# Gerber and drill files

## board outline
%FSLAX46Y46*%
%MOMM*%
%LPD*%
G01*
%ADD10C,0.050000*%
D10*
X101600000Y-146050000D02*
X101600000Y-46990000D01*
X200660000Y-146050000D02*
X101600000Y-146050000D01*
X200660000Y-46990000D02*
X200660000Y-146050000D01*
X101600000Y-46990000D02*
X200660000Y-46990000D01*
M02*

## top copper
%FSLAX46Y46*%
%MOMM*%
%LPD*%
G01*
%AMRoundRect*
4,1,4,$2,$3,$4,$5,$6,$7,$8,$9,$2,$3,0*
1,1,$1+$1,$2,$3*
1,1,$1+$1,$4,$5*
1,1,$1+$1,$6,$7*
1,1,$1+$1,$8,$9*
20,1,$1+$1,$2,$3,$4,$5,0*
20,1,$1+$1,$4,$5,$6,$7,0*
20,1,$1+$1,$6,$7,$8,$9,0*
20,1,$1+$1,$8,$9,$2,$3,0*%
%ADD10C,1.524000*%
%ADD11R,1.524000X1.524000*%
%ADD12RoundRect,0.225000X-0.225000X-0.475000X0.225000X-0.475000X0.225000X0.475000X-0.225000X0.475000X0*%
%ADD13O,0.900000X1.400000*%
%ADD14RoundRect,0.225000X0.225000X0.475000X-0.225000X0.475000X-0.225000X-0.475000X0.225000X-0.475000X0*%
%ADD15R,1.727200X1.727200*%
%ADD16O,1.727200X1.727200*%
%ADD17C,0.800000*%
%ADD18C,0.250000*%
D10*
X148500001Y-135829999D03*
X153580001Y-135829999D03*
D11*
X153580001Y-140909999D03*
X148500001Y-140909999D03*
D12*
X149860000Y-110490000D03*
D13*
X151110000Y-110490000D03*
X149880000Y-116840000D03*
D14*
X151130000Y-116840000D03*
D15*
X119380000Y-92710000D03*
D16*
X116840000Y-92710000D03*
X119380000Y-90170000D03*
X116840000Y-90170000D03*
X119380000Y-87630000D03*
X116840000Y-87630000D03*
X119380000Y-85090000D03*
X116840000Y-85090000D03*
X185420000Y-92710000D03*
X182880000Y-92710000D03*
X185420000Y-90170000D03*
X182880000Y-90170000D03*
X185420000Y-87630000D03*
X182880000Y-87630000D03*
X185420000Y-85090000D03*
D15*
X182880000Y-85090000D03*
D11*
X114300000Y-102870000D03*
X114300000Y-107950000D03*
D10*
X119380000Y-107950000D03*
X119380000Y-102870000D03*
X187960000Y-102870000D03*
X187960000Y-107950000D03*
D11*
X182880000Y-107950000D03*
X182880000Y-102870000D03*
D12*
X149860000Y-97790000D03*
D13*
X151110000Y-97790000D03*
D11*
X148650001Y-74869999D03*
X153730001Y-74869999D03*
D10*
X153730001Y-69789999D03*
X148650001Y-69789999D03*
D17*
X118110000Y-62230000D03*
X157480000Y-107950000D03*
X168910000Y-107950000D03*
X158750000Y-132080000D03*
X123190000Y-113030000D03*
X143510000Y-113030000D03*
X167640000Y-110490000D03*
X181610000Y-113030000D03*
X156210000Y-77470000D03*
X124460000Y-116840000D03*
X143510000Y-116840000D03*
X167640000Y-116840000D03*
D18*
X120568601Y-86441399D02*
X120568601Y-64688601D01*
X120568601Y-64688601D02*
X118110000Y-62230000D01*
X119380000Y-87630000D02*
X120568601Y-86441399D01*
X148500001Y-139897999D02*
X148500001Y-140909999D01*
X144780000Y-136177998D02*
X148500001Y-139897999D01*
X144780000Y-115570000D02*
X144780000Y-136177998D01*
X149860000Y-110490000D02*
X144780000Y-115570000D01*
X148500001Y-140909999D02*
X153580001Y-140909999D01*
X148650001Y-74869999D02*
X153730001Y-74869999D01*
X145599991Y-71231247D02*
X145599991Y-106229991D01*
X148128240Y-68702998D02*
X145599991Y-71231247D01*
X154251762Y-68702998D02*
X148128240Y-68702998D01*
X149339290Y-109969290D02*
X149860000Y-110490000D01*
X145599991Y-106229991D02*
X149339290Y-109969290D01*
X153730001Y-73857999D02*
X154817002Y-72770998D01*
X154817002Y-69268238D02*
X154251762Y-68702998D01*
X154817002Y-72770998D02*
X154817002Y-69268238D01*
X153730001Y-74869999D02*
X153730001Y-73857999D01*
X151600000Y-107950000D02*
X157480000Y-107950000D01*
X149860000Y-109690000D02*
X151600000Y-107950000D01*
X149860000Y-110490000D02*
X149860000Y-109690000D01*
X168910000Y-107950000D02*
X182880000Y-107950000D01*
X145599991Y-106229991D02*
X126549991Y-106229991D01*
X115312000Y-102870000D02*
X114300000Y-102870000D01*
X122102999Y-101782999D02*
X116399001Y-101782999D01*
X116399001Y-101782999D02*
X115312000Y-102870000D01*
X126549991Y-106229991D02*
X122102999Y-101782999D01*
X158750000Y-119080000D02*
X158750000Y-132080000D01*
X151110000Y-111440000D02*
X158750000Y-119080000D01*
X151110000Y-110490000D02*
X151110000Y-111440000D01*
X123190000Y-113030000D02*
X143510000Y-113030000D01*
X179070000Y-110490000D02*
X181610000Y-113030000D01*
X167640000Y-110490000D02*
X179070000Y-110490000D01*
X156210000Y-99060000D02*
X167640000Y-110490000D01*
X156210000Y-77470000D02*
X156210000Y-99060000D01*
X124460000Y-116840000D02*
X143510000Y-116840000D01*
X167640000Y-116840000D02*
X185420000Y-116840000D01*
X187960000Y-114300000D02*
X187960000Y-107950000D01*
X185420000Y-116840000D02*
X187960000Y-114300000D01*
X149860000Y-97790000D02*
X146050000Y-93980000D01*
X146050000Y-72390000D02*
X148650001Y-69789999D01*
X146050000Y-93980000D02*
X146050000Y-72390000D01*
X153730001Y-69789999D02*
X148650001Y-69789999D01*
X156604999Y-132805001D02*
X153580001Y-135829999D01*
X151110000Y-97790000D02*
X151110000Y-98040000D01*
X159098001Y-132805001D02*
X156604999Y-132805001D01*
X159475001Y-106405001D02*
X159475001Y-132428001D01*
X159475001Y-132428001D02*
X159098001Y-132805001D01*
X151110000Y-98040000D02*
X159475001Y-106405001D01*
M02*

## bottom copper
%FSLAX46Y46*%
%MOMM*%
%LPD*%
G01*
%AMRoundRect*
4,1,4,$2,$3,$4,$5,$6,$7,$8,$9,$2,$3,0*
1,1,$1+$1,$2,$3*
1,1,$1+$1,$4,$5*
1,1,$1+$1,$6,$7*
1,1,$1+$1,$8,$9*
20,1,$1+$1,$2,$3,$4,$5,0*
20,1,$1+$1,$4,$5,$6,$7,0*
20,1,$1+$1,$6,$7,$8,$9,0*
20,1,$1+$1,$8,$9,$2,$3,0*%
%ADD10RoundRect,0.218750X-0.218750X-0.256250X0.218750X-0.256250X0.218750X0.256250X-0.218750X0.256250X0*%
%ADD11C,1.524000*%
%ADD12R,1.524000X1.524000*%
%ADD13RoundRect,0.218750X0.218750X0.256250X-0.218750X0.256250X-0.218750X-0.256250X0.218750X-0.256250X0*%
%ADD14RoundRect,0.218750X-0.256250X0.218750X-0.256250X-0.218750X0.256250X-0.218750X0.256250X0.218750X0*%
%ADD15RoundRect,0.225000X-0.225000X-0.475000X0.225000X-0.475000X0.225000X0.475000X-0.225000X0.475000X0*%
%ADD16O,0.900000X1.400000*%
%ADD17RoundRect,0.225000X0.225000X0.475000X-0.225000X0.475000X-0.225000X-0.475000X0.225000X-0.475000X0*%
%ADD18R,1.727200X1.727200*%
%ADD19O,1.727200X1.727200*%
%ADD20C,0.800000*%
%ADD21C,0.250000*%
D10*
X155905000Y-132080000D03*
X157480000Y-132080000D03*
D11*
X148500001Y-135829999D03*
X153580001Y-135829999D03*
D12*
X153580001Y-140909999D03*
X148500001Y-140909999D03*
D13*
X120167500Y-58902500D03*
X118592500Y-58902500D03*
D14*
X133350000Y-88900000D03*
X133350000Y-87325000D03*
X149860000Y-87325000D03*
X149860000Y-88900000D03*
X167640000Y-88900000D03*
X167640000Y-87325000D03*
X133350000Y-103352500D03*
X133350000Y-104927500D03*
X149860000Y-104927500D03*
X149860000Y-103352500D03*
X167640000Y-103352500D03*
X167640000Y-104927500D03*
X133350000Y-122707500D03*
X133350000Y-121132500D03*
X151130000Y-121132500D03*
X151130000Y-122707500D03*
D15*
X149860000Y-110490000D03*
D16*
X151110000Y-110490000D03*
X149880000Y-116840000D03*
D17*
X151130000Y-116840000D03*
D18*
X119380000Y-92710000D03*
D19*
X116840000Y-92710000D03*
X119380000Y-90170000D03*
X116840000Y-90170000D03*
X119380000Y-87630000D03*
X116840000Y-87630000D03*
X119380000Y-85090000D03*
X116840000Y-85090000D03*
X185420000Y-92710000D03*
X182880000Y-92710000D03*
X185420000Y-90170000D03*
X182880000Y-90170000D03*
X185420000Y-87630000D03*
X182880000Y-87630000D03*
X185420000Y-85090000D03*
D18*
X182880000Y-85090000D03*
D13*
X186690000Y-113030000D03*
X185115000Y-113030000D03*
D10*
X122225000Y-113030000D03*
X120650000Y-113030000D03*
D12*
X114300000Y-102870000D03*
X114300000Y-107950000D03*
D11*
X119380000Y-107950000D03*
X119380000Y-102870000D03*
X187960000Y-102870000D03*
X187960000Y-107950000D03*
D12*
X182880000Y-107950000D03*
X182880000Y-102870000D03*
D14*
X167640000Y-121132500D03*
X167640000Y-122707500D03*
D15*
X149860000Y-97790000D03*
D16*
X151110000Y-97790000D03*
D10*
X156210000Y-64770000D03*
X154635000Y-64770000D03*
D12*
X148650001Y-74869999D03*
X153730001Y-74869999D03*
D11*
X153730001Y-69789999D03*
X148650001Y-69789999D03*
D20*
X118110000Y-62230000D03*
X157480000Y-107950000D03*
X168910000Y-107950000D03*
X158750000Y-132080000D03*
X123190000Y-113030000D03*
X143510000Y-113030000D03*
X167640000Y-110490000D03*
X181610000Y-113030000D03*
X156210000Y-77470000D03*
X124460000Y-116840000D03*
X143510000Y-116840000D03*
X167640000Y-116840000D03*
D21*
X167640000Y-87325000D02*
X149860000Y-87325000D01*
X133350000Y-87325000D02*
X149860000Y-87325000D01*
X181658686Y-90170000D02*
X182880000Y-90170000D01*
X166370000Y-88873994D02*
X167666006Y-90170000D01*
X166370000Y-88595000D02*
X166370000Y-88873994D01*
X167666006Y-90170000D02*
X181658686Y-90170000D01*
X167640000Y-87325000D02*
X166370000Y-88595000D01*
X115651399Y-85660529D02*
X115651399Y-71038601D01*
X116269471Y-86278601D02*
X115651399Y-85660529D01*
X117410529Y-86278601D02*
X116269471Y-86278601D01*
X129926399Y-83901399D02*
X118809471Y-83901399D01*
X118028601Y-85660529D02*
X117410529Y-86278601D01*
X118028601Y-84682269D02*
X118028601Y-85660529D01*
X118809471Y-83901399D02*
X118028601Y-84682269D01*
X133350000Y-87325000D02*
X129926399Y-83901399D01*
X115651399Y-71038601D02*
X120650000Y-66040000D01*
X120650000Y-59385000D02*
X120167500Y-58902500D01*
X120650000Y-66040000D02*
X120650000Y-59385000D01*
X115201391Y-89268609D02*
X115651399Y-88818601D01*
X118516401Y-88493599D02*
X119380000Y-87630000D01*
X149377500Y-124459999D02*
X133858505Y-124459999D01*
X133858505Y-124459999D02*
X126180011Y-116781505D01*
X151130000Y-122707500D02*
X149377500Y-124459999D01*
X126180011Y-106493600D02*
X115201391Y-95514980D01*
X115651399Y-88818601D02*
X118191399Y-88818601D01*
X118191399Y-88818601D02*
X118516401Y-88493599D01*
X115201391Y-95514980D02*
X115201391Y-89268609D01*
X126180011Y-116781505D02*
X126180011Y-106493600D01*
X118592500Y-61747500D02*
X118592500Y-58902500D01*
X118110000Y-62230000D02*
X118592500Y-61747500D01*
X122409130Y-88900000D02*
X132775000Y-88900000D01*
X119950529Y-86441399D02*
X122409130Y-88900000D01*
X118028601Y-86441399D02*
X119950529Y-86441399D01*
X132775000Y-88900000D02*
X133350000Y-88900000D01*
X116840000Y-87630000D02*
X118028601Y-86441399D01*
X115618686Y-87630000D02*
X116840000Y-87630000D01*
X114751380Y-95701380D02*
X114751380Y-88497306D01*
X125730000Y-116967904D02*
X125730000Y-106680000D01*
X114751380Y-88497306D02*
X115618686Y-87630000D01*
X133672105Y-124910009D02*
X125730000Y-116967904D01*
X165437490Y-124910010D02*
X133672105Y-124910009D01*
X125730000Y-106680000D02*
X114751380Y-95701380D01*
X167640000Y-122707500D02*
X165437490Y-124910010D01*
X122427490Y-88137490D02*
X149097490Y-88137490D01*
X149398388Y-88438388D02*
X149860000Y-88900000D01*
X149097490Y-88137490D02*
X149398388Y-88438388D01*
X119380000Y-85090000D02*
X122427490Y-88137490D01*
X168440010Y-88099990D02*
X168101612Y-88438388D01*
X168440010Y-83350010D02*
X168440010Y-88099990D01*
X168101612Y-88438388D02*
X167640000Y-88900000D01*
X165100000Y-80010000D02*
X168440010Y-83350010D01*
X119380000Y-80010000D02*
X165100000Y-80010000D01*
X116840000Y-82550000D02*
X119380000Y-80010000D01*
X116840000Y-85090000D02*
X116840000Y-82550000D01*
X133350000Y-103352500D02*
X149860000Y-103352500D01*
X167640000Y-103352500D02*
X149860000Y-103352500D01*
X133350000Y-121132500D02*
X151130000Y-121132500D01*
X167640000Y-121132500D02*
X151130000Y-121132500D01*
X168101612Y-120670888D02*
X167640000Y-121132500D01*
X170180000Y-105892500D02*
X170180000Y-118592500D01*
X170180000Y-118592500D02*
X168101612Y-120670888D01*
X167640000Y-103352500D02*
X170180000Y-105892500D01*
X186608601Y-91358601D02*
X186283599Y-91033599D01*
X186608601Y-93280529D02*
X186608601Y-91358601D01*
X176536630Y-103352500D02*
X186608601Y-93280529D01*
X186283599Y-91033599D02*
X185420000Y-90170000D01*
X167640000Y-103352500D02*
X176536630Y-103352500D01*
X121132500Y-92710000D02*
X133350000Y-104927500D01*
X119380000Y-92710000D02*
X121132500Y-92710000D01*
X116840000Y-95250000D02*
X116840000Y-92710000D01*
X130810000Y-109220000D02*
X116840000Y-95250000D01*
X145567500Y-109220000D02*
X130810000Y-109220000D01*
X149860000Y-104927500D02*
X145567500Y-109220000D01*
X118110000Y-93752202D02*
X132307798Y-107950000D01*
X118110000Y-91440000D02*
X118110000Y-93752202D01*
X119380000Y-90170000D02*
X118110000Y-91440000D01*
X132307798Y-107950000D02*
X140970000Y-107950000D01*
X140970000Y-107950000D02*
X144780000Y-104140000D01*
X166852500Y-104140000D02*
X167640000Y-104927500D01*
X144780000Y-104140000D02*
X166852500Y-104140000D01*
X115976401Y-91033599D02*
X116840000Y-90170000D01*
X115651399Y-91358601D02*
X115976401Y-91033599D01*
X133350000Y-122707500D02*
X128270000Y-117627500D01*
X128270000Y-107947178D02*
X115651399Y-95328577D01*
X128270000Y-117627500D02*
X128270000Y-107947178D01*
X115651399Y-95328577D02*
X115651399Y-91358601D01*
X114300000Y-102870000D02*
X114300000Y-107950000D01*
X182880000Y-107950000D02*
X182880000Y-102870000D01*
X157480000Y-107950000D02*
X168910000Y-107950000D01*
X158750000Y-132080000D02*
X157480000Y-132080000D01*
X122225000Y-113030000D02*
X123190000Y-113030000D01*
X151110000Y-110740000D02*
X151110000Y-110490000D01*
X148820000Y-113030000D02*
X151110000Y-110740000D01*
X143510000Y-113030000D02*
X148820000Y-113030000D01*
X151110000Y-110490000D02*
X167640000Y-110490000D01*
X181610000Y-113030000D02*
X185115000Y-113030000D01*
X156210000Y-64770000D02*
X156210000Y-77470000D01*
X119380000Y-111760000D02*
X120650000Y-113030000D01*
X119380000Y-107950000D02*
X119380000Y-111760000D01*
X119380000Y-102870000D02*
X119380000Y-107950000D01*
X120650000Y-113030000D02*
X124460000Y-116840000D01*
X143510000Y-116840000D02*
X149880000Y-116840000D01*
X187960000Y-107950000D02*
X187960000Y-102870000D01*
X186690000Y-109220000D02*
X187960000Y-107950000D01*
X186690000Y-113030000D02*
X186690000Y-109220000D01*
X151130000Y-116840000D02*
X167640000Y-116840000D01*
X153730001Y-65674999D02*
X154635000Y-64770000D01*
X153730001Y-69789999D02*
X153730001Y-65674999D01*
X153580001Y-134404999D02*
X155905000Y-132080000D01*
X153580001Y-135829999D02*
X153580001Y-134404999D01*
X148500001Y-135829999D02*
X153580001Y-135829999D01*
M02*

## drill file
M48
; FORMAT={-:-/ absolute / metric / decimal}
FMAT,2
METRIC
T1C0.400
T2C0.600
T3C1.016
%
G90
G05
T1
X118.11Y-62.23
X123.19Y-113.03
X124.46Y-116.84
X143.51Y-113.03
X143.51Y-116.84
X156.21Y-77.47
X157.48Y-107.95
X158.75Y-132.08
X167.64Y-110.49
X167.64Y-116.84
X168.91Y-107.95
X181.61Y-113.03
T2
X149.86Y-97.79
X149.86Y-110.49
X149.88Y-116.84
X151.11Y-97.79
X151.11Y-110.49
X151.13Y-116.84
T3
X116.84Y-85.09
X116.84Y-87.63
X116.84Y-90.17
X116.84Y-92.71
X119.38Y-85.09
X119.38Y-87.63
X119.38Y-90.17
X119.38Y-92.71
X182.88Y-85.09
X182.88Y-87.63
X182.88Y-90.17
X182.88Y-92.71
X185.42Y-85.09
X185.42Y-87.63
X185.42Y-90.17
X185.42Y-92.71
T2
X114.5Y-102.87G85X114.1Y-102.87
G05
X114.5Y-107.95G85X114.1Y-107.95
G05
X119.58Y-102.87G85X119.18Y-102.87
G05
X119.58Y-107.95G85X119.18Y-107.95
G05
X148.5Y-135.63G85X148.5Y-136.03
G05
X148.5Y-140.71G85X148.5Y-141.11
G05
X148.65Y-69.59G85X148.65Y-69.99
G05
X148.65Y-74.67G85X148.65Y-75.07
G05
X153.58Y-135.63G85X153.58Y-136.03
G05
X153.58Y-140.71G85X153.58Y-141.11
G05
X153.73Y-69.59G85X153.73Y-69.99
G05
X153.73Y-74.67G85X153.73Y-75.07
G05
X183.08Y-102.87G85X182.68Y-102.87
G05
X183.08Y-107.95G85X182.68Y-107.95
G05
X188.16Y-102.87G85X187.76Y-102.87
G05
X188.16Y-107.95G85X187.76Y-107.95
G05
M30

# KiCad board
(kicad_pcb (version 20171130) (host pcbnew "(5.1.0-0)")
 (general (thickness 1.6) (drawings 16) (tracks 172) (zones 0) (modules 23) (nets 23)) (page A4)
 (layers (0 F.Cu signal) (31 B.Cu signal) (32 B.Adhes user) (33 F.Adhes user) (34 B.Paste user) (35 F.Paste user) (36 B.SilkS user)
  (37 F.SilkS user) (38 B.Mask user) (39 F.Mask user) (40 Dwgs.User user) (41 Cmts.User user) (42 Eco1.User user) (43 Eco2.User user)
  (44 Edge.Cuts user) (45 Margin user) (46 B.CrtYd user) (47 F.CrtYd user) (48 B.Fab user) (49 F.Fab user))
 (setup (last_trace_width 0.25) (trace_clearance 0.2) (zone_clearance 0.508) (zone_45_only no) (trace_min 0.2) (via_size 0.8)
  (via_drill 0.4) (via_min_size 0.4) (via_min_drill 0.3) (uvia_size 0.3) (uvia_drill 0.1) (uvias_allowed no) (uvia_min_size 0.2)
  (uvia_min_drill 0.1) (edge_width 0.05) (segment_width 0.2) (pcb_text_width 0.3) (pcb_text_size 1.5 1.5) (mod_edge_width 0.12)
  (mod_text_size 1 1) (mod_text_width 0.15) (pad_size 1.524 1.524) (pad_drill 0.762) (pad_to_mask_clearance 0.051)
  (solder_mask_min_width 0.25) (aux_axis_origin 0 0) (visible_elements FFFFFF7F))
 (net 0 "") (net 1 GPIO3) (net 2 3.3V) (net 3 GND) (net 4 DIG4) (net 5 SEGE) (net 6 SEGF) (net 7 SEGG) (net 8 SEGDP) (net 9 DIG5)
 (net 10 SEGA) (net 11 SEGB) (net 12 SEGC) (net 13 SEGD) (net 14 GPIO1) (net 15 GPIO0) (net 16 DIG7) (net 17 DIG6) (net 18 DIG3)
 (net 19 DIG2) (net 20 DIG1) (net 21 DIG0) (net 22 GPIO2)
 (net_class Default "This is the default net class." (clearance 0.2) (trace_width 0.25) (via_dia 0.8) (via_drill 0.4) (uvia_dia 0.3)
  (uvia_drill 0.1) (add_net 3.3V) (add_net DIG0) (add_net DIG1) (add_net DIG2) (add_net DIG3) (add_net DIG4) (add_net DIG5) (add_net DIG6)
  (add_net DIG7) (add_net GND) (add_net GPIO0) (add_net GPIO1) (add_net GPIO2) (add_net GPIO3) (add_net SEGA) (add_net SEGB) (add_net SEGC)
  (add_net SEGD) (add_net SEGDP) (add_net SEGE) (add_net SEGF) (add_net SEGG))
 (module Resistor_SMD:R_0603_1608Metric (layer B.Cu) (at 156.6925 132.08)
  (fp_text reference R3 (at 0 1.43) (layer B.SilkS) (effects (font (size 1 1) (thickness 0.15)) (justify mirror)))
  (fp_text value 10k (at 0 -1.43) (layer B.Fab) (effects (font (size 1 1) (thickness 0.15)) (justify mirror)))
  (pad 1 smd roundrect (at -0.7875 0) (size 0.875 0.95) (layers B.Cu B.Paste B.Mask) (roundrect_rratio 0.25) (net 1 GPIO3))
  (pad 2 smd roundrect (at 0.7875 0) (size 0.875 0.95) (layers B.Cu B.Paste B.Mask) (roundrect_rratio 0.25) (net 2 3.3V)))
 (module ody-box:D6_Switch (layer B.Cu) (at 151.040001 138.369999)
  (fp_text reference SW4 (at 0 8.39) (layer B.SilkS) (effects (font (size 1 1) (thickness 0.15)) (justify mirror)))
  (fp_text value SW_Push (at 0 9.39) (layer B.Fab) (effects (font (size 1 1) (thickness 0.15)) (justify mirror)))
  (pad 2 thru_hole circle (at -2.54 -2.54) (size 1.524 1.524) (drill oval 0.6 1) (layers *.Cu *.Mask) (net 1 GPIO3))
  (pad 2 thru_hole circle (at 2.54 -2.54) (size 1.524 1.524) (drill oval 0.6 1) (layers *.Cu *.Mask) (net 1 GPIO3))
  (pad 1 thru_hole rect (at 2.54 2.54) (size 1.524 1.524) (drill oval 0.6 1) (layers *.Cu *.Mask) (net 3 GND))
  (pad 1 thru_hole rect (at -2.54 2.54) (size 1.524 1.524) (drill oval 0.6 1) (layers *.Cu *.Mask) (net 3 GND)))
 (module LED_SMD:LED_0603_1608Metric (layer B.Cu) (at 119.38 58.9025 180)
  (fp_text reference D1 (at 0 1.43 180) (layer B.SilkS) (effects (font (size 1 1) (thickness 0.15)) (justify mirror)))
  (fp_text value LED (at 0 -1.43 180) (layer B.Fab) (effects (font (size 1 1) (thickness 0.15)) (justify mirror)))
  (pad 1 smd roundrect (at -0.7875 0 180) (size 0.875 0.95) (layers B.Cu B.Paste B.Mask) (roundrect_rratio 0.25) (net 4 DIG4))
  (pad 2 smd roundrect (at 0.7875 0 180) (size 0.875 0.95) (layers B.Cu B.Paste B.Mask) (roundrect_rratio 0.25) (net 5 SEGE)))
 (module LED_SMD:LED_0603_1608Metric (layer B.Cu) (at 133.35 88.1125 270)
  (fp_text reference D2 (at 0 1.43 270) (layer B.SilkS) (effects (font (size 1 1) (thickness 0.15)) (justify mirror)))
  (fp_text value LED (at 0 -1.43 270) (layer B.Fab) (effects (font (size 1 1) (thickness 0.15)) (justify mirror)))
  (pad 2 smd roundrect (at 0.7875 0 270) (size 0.875 0.95) (layers B.Cu B.Paste B.Mask) (roundrect_rratio 0.25) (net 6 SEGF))
  (pad 1 smd roundrect (at -0.7875 0 270) (size 0.875 0.95) (layers B.Cu B.Paste B.Mask) (roundrect_rratio 0.25) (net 4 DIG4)))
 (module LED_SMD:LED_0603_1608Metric (layer B.Cu) (at 149.86 88.1125 270)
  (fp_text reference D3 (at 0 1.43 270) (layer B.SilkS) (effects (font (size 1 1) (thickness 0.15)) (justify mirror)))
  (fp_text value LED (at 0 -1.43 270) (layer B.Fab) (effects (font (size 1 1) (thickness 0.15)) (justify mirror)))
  (pad 1 smd roundrect (at -0.7875 0 270) (size 0.875 0.95) (layers B.Cu B.Paste B.Mask) (roundrect_rratio 0.25) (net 4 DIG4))
  (pad 2 smd roundrect (at 0.7875 0 270) (size 0.875 0.95) (layers B.Cu B.Paste B.Mask) (roundrect_rratio 0.25) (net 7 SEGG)))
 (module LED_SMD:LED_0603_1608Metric (layer B.Cu) (at 167.64 88.1125 270)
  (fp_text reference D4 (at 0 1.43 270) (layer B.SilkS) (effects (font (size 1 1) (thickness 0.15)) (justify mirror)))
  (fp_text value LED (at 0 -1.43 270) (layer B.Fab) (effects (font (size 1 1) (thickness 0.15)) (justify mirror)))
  (pad 2 smd roundrect (at 0.7875 0 270) (size 0.875 0.95) (layers B.Cu B.Paste B.Mask) (roundrect_rratio 0.25) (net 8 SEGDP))
  (pad 1 smd roundrect (at -0.7875 0 270) (size 0.875 0.95) (layers B.Cu B.Paste B.Mask) (roundrect_rratio 0.25) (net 4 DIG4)))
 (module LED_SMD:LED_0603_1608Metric (layer B.Cu) (at 133.35 104.14 270)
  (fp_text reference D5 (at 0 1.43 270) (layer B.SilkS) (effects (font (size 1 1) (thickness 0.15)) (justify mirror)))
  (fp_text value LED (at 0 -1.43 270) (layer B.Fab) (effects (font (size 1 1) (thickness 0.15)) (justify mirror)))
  (pad 1 smd roundrect (at -0.7875 0 270) (size 0.875 0.95) (layers B.Cu B.Paste B.Mask) (roundrect_rratio 0.25) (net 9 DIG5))
  (pad 2 smd roundrect (at 0.7875 0 270) (size 0.875 0.95) (layers B.Cu B.Paste B.Mask) (roundrect_rratio 0.25) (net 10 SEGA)))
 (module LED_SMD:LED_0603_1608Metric (layer B.Cu) (at 149.86 104.14 270)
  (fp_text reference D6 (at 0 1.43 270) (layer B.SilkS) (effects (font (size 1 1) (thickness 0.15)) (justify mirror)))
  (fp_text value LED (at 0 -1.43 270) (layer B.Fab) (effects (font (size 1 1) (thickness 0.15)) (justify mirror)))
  (pad 2 smd roundrect (at 0.7875 0 270) (size 0.875 0.95) (layers B.Cu B.Paste B.Mask) (roundrect_rratio 0.25) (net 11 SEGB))
  (pad 1 smd roundrect (at -0.7875 0 270) (size 0.875 0.95) (layers B.Cu B.Paste B.Mask) (roundrect_rratio 0.25) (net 9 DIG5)))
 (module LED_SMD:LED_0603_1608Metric (layer B.Cu) (at 167.64 104.14 270)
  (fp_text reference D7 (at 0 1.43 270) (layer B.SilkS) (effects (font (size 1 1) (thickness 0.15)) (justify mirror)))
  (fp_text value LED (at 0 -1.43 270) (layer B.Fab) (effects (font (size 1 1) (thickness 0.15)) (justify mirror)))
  (pad 1 smd roundrect (at -0.7875 0 270) (size 0.875 0.95) (layers B.Cu B.Paste B.Mask) (roundrect_rratio 0.25) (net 9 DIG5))
  (pad 2 smd roundrect (at 0.7875 0 270) (size 0.875 0.95) (layers B.Cu B.Paste B.Mask) (roundrect_rratio 0.25) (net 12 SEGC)))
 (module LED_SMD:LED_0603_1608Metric (layer B.Cu) (at 133.35 121.92 270)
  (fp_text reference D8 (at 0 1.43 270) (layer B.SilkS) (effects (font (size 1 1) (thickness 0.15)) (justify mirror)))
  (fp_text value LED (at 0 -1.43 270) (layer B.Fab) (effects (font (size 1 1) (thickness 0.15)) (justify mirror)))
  (pad 2 smd roundrect (at 0.7875 0 270) (size 0.875 0.95) (layers B.Cu B.Paste B.Mask) (roundrect_rratio 0.25) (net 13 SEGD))
  (pad 1 smd roundrect (at -0.7875 0 270) (size 0.875 0.95) (layers B.Cu B.Paste B.Mask) (roundrect_rratio 0.25) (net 9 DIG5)))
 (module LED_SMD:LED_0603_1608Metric (layer B.Cu) (at 151.13 121.92 270)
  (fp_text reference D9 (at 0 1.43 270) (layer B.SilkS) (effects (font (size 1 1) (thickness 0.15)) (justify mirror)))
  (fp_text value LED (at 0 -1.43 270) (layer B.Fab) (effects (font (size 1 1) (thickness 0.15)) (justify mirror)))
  (pad 1 smd roundrect (at -0.7875 0 270) (size 0.875 0.95) (layers B.Cu B.Paste B.Mask) (roundrect_rratio 0.25) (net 9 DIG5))
  (pad 2 smd roundrect (at 0.7875 0 270) (size 0.875 0.95) (layers B.Cu B.Paste B.Mask) (roundrect_rratio 0.25) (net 5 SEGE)))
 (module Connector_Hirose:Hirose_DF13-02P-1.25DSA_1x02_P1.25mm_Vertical (layer F.Cu) (at 149.86 110.49)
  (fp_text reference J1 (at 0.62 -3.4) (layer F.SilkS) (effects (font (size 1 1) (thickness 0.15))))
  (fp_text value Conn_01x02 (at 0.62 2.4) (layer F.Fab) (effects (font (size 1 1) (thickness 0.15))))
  (pad 1 thru_hole roundrect (at 0 0) (size 0.9 1.4) (drill 0.6) (layers *.Cu *.Mask) (roundrect_rratio 0.25) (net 3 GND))
  (pad 2 thru_hole oval (at 1.25 0) (size 0.9 1.4) (drill 0.6) (layers *.Cu *.Mask) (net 2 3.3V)))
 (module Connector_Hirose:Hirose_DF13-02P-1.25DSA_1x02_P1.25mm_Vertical (layer F.Cu) (at 151.13 116.84 180)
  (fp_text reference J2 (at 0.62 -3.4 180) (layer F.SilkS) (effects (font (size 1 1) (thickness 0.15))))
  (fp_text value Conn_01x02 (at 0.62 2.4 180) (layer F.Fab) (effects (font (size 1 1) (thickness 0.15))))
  (pad 2 thru_hole oval (at 1.25 0 180) (size 0.9 1.4) (drill 0.6) (layers *.Cu *.Mask) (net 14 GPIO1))
  (pad 1 thru_hole roundrect (at 0 0 180) (size 0.9 1.4) (drill 0.6) (layers *.Cu *.Mask) (roundrect_rratio 0.25) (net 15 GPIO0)))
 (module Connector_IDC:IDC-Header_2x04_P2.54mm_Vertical (layer F.Cu) (at 119.38 92.71 180)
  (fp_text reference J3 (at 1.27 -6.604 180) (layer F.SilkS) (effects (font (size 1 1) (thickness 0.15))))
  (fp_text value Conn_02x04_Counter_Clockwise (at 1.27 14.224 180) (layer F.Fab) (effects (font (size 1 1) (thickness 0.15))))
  (pad 1 thru_hole rect (at 0 0 180) (size 1.7272 1.7272) (drill 1.016) (layers *.Cu *.Mask) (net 10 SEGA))
  (pad 2 thru_hole oval (at 2.54 0 180) (size 1.7272 1.7272) (drill 1.016) (layers *.Cu *.Mask) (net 11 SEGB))
  (pad 3 thru_hole oval (at 0 2.54 180) (size 1.7272 1.7272) (drill 1.016) (layers *.Cu *.Mask) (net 12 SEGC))
  (pad 4 thru_hole oval (at 2.54 2.54 180) (size 1.7272 1.7272) (drill 1.016) (layers *.Cu *.Mask) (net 13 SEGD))
  (pad 5 thru_hole oval (at 0 5.08 180) (size 1.7272 1.7272) (drill 1.016) (layers *.Cu *.Mask) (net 5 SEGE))
  (pad 6 thru_hole oval (at 2.54 5.08 180) (size 1.7272 1.7272) (drill 1.016) (layers *.Cu *.Mask) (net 6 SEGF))
  (pad 7 thru_hole oval (at 0 7.62 180) (size 1.7272 1.7272) (drill 1.016) (layers *.Cu *.Mask) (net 7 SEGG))
  (pad 8 thru_hole oval (at 2.54 7.62 180) (size 1.7272 1.7272) (drill 1.016) (layers *.Cu *.Mask) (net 8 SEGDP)))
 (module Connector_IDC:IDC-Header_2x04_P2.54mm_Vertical (layer F.Cu) (at 182.88 85.09)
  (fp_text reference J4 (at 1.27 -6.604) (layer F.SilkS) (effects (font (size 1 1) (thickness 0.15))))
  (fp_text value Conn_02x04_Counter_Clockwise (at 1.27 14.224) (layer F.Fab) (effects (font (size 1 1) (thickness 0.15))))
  (pad 8 thru_hole oval (at 2.54 7.62) (size 1.7272 1.7272) (drill 1.016) (layers *.Cu *.Mask) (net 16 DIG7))
  (pad 7 thru_hole oval (at 0 7.62) (size 1.7272 1.7272) (drill 1.016) (layers *.Cu *.Mask) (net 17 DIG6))
  (pad 6 thru_hole oval (at 2.54 5.08) (size 1.7272 1.7272) (drill 1.016) (layers *.Cu *.Mask) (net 9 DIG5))
  (pad 5 thru_hole oval (at 0 5.08) (size 1.7272 1.7272) (drill 1.016) (layers *.Cu *.Mask) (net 4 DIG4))
  (pad 4 thru_hole oval (at 2.54 2.54) (size 1.7272 1.7272) (drill 1.016) (layers *.Cu *.Mask) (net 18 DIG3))
  (pad 3 thru_hole oval (at 0 2.54) (size 1.7272 1.7272) (drill 1.016) (layers *.Cu *.Mask) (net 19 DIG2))
  (pad 2 thru_hole oval (at 2.54 0) (size 1.7272 1.7272) (drill 1.016) (layers *.Cu *.Mask) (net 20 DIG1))
  (pad 1 thru_hole rect (at 0 0) (size 1.7272 1.7272) (drill 1.016) (layers *.Cu *.Mask) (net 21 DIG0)))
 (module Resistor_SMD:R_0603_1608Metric (layer B.Cu) (at 185.9025 113.03 180)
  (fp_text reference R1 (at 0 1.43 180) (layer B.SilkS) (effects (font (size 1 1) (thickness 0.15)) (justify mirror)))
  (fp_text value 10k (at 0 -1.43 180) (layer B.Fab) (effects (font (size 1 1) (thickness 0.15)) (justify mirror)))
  (pad 1 smd roundrect (at -0.7875 0 180) (size 0.875 0.95) (layers B.Cu B.Paste B.Mask) (roundrect_rratio 0.25) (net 15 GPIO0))
  (pad 2 smd roundrect (at 0.7875 0 180) (size 0.875 0.95) (layers B.Cu B.Paste B.Mask) (roundrect_rratio 0.25) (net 2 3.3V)))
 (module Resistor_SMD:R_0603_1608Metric (layer B.Cu) (at 121.4375 113.03)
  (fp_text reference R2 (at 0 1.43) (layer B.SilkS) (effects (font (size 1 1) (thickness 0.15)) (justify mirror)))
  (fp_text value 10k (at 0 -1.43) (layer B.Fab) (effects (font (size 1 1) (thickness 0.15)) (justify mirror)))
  (pad 2 smd roundrect (at 0.7875 0) (size 0.875 0.95) (layers B.Cu B.Paste B.Mask) (roundrect_rratio 0.25) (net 2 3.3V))
  (pad 1 smd roundrect (at -0.7875 0) (size 0.875 0.95) (layers B.Cu B.Paste B.Mask) (roundrect_rratio 0.25) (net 14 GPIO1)))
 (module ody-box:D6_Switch (layer B.Cu) (at 116.84 105.41 270)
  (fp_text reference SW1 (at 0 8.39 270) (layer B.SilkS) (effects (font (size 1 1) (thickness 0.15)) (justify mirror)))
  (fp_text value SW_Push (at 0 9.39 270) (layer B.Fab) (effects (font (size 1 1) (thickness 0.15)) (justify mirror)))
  (pad 1 thru_hole rect (at -2.54 2.54 270) (size 1.524 1.524) (drill oval 0.6 1) (layers *.Cu *.Mask) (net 3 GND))
  (pad 1 thru_hole rect (at 2.54 2.54 270) (size 1.524 1.524) (drill oval 0.6 1) (layers *.Cu *.Mask) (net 3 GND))
  (pad 2 thru_hole circle (at 2.54 -2.54 270) (size 1.524 1.524) (drill oval 0.6 1) (layers *.Cu *.Mask) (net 14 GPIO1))
  (pad 2 thru_hole circle (at -2.54 -2.54 270) (size 1.524 1.524) (drill oval 0.6 1) (layers *.Cu *.Mask) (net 14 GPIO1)))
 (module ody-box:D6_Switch (layer B.Cu) (at 185.42 105.41 270)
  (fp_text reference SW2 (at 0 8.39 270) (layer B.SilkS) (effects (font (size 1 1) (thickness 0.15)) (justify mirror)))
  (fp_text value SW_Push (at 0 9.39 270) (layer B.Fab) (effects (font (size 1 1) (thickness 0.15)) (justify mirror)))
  (pad 2 thru_hole circle (at -2.54 -2.54 270) (size 1.524 1.524) (drill oval 0.6 1) (layers *.Cu *.Mask) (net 15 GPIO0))
  (pad 2 thru_hole circle (at 2.54 -2.54 270) (size 1.524 1.524) (drill oval 0.6 1) (layers *.Cu *.Mask) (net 15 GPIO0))
  (pad 1 thru_hole rect (at 2.54 2.54 270) (size 1.524 1.524) (drill oval 0.6 1) (layers *.Cu *.Mask) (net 3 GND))
  (pad 1 thru_hole rect (at -2.54 2.54 270) (size 1.524 1.524) (drill oval 0.6 1) (layers *.Cu *.Mask) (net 3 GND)))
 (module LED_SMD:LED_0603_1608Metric (layer B.Cu) (at 167.64 121.92 270)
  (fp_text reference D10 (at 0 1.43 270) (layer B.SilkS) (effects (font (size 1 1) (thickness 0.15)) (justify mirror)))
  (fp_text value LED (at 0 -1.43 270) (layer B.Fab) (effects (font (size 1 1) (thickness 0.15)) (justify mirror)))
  (pad 1 smd roundrect (at -0.7875 0 270) (size 0.875 0.95) (layers B.Cu B.Paste B.Mask) (roundrect_rratio 0.25) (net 9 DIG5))
  (pad 2 smd roundrect (at 0.7875 0 270) (size 0.875 0.95) (layers B.Cu B.Paste B.Mask) (roundrect_rratio 0.25) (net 6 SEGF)))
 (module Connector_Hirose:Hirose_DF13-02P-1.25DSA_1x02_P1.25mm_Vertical (layer F.Cu) (at 149.86 97.79)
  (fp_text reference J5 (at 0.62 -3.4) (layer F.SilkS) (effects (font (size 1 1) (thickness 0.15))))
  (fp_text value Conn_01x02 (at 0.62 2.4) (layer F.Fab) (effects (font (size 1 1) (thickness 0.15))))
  (pad 1 thru_hole roundrect (at 0 0) (size 0.9 1.4) (drill 0.6) (layers *.Cu *.Mask) (roundrect_rratio 0.25) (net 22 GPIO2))
  (pad 2 thru_hole oval (at 1.25 0) (size 0.9 1.4) (drill 0.6) (layers *.Cu *.Mask) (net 1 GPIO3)))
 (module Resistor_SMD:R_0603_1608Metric (layer B.Cu) (at 155.4225 64.77)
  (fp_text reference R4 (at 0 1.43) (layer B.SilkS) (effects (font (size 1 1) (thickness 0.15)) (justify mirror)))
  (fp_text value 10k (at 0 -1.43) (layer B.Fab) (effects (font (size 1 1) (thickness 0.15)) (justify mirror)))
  (pad 2 smd roundrect (at 0.7875 0) (size 0.875 0.95) (layers B.Cu B.Paste B.Mask) (roundrect_rratio 0.25) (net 2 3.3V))
  (pad 1 smd roundrect (at -0.7875 0) (size 0.875 0.95) (layers B.Cu B.Paste B.Mask) (roundrect_rratio 0.25) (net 22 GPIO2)))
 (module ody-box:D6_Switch (layer B.Cu) (at 151.190001 72.329999)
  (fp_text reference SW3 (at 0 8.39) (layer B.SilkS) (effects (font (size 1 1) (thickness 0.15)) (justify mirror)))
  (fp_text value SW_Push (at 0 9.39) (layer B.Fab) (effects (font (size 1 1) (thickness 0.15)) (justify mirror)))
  (pad 1 thru_hole rect (at -2.54 2.54) (size 1.524 1.524) (drill oval 0.6 1) (layers *.Cu *.Mask) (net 3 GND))
  (pad 1 thru_hole rect (at 2.54 2.54) (size 1.524 1.524) (drill oval 0.6 1) (layers *.Cu *.Mask) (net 3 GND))
  (pad 2 thru_hole circle (at 2.54 -2.54) (size 1.524 1.524) (drill oval 0.6 1) (layers *.Cu *.Mask) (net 22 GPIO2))
  (pad 2 thru_hole circle (at -2.54 -2.54) (size 1.524 1.524) (drill oval 0.6 1) (layers *.Cu *.Mask) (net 22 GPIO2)))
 (gr_line (start 101.6 146.05) (end 101.6 46.99) (layer Edge.Cuts) (width 0.05))
 (gr_line (start 200.66 146.05) (end 101.6 146.05) (layer Edge.Cuts) (width 0.05))
 (gr_line (start 200.66 46.99) (end 200.66 146.05) (layer Edge.Cuts) (width 0.05))
 (gr_line (start 101.6 46.99) (end 200.66 46.99) (layer Edge.Cuts) (width 0.05))
 (segment (start 167.64 87.325) (end 149.86 87.325) (width 0.25) (layer B.Cu) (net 4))
 (segment (start 133.35 87.325) (end 149.86 87.325) (width 0.25) (layer B.Cu) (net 4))
 (segment (start 181.658686 90.17) (end 182.88 90.17) (width 0.25) (layer B.Cu) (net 4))
 (segment (start 166.37 88.873994) (end 167.666006 90.17) (width 0.25) (layer B.Cu) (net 4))
 (segment (start 166.37 88.595) (end 166.37 88.873994) (width 0.25) (layer B.Cu) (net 4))
 (segment (start 167.666006 90.17) (end 181.658686 90.17) (width 0.25) (layer B.Cu) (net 4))
 (segment (start 167.64 87.325) (end 166.37 88.595) (width 0.25) (layer B.Cu) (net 4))
 (segment (start 115.651399 85.660529) (end 115.651399 71.038601) (width 0.25) (layer B.Cu) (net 4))
 (segment (start 116.269471 86.278601) (end 115.651399 85.660529) (width 0.25) (layer B.Cu) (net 4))
 (segment (start 117.410529 86.278601) (end 116.269471 86.278601) (width 0.25) (layer B.Cu) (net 4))
 (segment (start 129.926399 83.901399) (end 118.809471 83.901399) (width 0.25) (layer B.Cu) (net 4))
 (segment (start 118.028601 85.660529) (end 117.410529 86.278601) (width 0.25) (layer B.Cu) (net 4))
 (segment (start 118.028601 84.682269) (end 118.028601 85.660529) (width 0.25) (layer B.Cu) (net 4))
 (segment (start 118.809471 83.901399) (end 118.028601 84.682269) (width 0.25) (layer B.Cu) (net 4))
 (segment (start 133.35 87.325) (end 129.926399 83.901399) (width 0.25) (layer B.Cu) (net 4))
 (segment (start 115.651399 71.038601) (end 120.65 66.04) (width 0.25) (layer B.Cu) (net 4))
 (segment (start 120.65 59.385) (end 120.1675 58.9025) (width 0.25) (layer B.Cu) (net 4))
 (segment (start 120.65 66.04) (end 120.65 59.385) (width 0.25) (layer B.Cu) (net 4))
 (segment (start 115.201391 89.268609) (end 115.651399 88.818601) (width 0.25) (layer B.Cu) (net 5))
 (segment (start 118.516401 88.493599) (end 119.38 87.63) (width 0.25) (layer B.Cu) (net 5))
 (segment (start 149.3775 124.459999) (end 133.858505 124.459999) (width 0.25) (layer B.Cu) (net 5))
 (segment (start 133.858505 124.459999) (end 126.180011 116.781505) (width 0.25) (layer B.Cu) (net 5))
 (segment (start 151.13 122.7075) (end 149.3775 124.459999) (width 0.25) (layer B.Cu) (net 5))
 (segment (start 126.180011 106.4936) (end 115.201391 95.51498) (width 0.25) (layer B.Cu) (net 5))
 (segment (start 115.651399 88.818601) (end 118.191399 88.818601) (width 0.25) (layer B.Cu) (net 5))
 (segment (start 118.191399 88.818601) (end 118.516401 88.493599) (width 0.25) (layer B.Cu) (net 5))
 (segment (start 115.201391 95.51498) (end 115.201391 89.268609) (width 0.25) (layer B.Cu) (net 5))
 (segment (start 126.180011 116.781505) (end 126.180011 106.4936) (width 0.25) (layer B.Cu) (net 5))
 (segment (start 120.568601 86.441399) (end 120.568601 64.688601) (width 0.25) (layer F.Cu) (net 5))
 (via (at 118.11 62.23) (size 0.8) (drill 0.4) (layers F.Cu B.Cu) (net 5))
 (segment (start 120.568601 64.688601) (end 118.11 62.23) (width 0.25) (layer F.Cu) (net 5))
 (segment (start 119.38 87.63) (end 120.568601 86.441399) (width 0.25) (layer F.Cu) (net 5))
 (segment (start 118.5925 61.7475) (end 118.5925 58.9025) (width 0.25) (layer B.Cu) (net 5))
 (segment (start 118.11 62.23) (end 118.5925 61.7475) (width 0.25) (layer B.Cu) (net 5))
 (segment (start 122.40913 88.9) (end 132.775 88.9) (width 0.25) (layer B.Cu) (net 6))
 (segment (start 119.950529 86.441399) (end 122.40913 88.9) (width 0.25) (layer B.Cu) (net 6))
 (segment (start 118.028601 86.441399) (end 119.950529 86.441399) (width 0.25) (layer B.Cu) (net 6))
 (segment (start 132.775 88.9) (end 133.35 88.9) (width 0.25) (layer B.Cu) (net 6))
 (segment (start 116.84 87.63) (end 118.028601 86.441399) (width 0.25) (layer B.Cu) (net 6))
 (segment (start 115.618686 87.63) (end 116.84 87.63) (width 0.25) (layer B.Cu) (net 6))
 (segment (start 114.75138 95.70138) (end 114.75138 88.497306) (width 0.25) (layer B.Cu) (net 6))
 (segment (start 125.73 116.967904) (end 125.73 106.68) (width 0.25) (layer B.Cu) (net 6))
 (segment (start 114.75138 88.497306) (end 115.618686 87.63) (width 0.25) (layer B.Cu) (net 6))
 (segment (start 133.672105 124.910009) (end 125.73 116.967904) (width 0.25) (layer B.Cu) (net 6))
 (segment (start 165.43749 124.91001) (end 133.672105 124.910009) (width 0.25) (layer B.Cu) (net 6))
 (segment (start 125.73 106.68) (end 114.75138 95.70138) (width 0.25) (layer B.Cu) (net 6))
 (segment (start 167.64 122.7075) (end 165.43749 124.91001) (width 0.25) (layer B.Cu) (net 6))
 (segment (start 122.42749 88.13749) (end 149.09749 88.13749) (width 0.25) (layer B.Cu) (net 7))
 (segment (start 149.398388 88.438388) (end 149.86 88.9) (width 0.25) (layer B.Cu) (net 7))
 (segment (start 149.09749 88.13749) (end 149.398388 88.438388) (width 0.25) (layer B.Cu) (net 7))
 (segment (start 119.38 85.09) (end 122.42749 88.13749) (width 0.25) (layer B.Cu) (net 7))
 (segment (start 168.44001 88.09999) (end 168.101612 88.438388) (width 0.25) (layer B.Cu) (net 8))
 (segment (start 168.44001 83.35001) (end 168.44001 88.09999) (width 0.25) (layer B.Cu) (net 8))
 (segment (start 168.101612 88.438388) (end 167.64 88.9) (width 0.25) (layer B.Cu) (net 8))
 (segment (start 165.1 80.01) (end 168.44001 83.35001) (width 0.25) (layer B.Cu) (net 8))
 (segment (start 119.38 80.01) (end 165.1 80.01) (width 0.25) (layer B.Cu) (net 8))
 (segment (start 116.84 82.55) (end 119.38 80.01) (width 0.25) (layer B.Cu) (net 8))
 (segment (start 116.84 85.09) (end 116.84 82.55) (width 0.25) (layer B.Cu) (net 8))
 (segment (start 133.35 103.3525) (end 149.86 103.3525) (width 0.25) (layer B.Cu) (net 9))
 (segment (start 167.64 103.3525) (end 149.86 103.3525) (width 0.25) (layer B.Cu) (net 9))
 (segment (start 133.35 121.1325) (end 151.13 121.1325) (width 0.25) (layer B.Cu) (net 9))
 (segment (start 167.64 121.1325) (end 151.13 121.1325) (width 0.25) (layer B.Cu) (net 9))
 (segment (start 168.101612 120.670888) (end 167.64 121.1325) (width 0.25) (layer B.Cu) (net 9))
 (segment (start 170.18 105.8925) (end 170.18 118.5925) (width 0.25) (layer B.Cu) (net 9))
 (segment (start 170.18 118.5925) (end 168.101612 120.670888) (width 0.25) (layer B.Cu) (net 9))
 (segment (start 167.64 103.3525) (end 170.18 105.8925) (width 0.25) (layer B.Cu) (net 9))
 (segment (start 186.608601 91.358601) (end 186.283599 91.033599) (width 0.25) (layer B.Cu) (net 9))
 (segment (start 186.608601 93.280529) (end 186.608601 91.358601) (width 0.25) (layer B.Cu) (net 9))
 (segment (start 176.53663 103.3525) (end 186.608601 93.280529) (width 0.25) (layer B.Cu) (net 9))
 (segment (start 186.283599 91.033599) (end 185.42 90.17) (width 0.25) (layer B.Cu) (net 9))
 (segment (start 167.64 103.3525) (end 176.53663 103.3525) (width 0.25) (layer B.Cu) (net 9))
 (segment (start 121.1325 92.71) (end 133.35 104.9275) (width 0.25) (layer B.Cu) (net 10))
 (segment (start 119.38 92.71) (end 121.1325 92.71) (width 0.25) (layer B.Cu) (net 10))
 (segment (start 116.84 95.25) (end 116.84 92.71) (width 0.25) (layer B.Cu) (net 11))
 (segment (start 130.81 109.22) (end 116.84 95.25) (width 0.25) (layer B.Cu) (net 11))
 (segment (start 145.5675 109.22) (end 130.81 109.22) (width 0.25) (layer B.Cu) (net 11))
 (segment (start 149.86 104.9275) (end 145.5675 109.22) (width 0.25) (layer B.Cu) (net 11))
 (segment (start 118.11 93.752202) (end 132.307798 107.95) (width 0.25) (layer B.Cu) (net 12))
 (segment (start 118.11 91.44) (end 118.11 93.752202) (width 0.25) (layer B.Cu) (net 12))
 (segment (start 119.38 90.17) (end 118.11 91.44) (width 0.25) (layer B.Cu) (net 12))
 (segment (start 132.307798 107.95) (end 140.97 107.95) (width 0.25) (layer B.Cu) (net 12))
 (segment (start 140.97 107.95) (end 144.78 104.14) (width 0.25) (layer B.Cu) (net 12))
 (segment (start 166.8525 104.14) (end 167.64 104.9275) (width 0.25) (layer B.Cu) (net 12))
 (segment (start 144.78 104.14) (end 166.8525 104.14) (width 0.25) (layer B.Cu) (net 12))
 (segment (start 115.976401 91.033599) (end 116.84 90.17) (width 0.25) (layer B.Cu) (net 13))
 (segment (start 115.651399 91.358601) (end 115.976401 91.033599) (width 0.25) (layer B.Cu) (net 13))
 (segment (start 133.35 122.7075) (end 128.27 117.6275) (width 0.25) (layer B.Cu) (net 13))
 (segment (start 128.27 107.947178) (end 115.651399 95.328577) (width 0.25) (layer B.Cu) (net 13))
 (segment (start 128.27 117.6275) (end 128.27 107.947178) (width 0.25) (layer B.Cu) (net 13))
 (segment (start 115.651399 95.328577) (end 115.651399 91.358601) (width 0.25) (layer B.Cu) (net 13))
 (segment (start 114.3 102.87) (end 114.3 107.95) (width 0.25) (layer B.Cu) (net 3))
 (segment (start 182.88 107.95) (end 182.88 102.87) (width 0.25) (layer B.Cu) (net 3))
 (segment (start 148.500001 139.897999) (end 148.500001 140.909999) (width 0.25) (layer F.Cu) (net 3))
 (segment (start 144.78 136.177998) (end 148.500001 139.897999) (width 0.25) (layer F.Cu) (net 3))
 (segment (start 144.78 115.57) (end 144.78 136.177998) (width 0.25) (layer F.Cu) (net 3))
 (segment (start 149.86 110.49) (end 144.78 115.57) (width 0.25) (layer F.Cu) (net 3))
 (segment (start 148.500001 140.909999) (end 153.580001 140.909999) (width 0.25) (layer F.Cu) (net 3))
 (segment (start 148.650001 74.869999) (end 153.730001 74.869999) (width 0.25) (layer F.Cu) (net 3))
 (segment (start 145.599991 71.231247) (end 145.599991 106.229991) (width 0.25) (layer F.Cu) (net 3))
 (segment (start 148.12824 68.702998) (end 145.599991 71.231247) (width 0.25) (layer F.Cu) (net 3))
 (segment (start 154.251762 68.702998) (end 148.12824 68.702998) (width 0.25) (layer F.Cu) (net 3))
 (segment (start 149.33929 109.96929) (end 149.86 110.49) (width 0.25) (layer F.Cu) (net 3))
 (segment (start 145.599991 106.229991) (end 149.33929 109.96929) (width 0.25) (layer F.Cu) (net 3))
 (segment (start 153.730001 73.857999) (end 154.817002 72.770998) (width 0.25) (layer F.Cu) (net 3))
 (segment (start 154.817002 69.268238) (end 154.251762 68.702998) (width 0.25) (layer F.Cu) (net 3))
 (segment (start 154.817002 72.770998) (end 154.817002 69.268238) (width 0.25) (layer F.Cu) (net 3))
 (segment (start 153.730001 74.869999) (end 153.730001 73.857999) (width 0.25) (layer F.Cu) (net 3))
 (via (at 157.48 107.95) (size 0.8) (drill 0.4) (layers F.Cu B.Cu) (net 3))
 (segment (start 151.6 107.95) (end 157.48 107.95) (width 0.25) (layer F.Cu) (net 3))
 (segment (start 149.86 109.69) (end 151.6 107.95) (width 0.25) (layer F.Cu) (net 3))
 (segment (start 149.86 110.49) (end 149.86 109.69) (width 0.25) (layer F.Cu) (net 3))
 (via (at 168.91 107.95) (size 0.8) (drill 0.4) (layers F.Cu B.Cu) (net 3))
 (segment (start 157.48 107.95) (end 168.91 107.95) (width 0.25) (layer B.Cu) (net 3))
 (segment (start 168.91 107.95) (end 182.88 107.95) (width 0.25) (layer F.Cu) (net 3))
 (segment (start 145.599991 106.229991) (end 126.549991 106.229991) (width 0.25) (layer F.Cu) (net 3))
 (segment (start 115.312 102.87) (end 114.3 102.87) (width 0.25) (layer F.Cu) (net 3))
 (segment (start 122.102999 101.782999) (end 116.399001 101.782999) (width 0.25) (layer F.Cu) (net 3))
 (segment (start 116.399001 101.782999) (end 115.312 102.87) (width 0.25) (layer F.Cu) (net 3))
 (segment (start 126.549991 106.229991) (end 122.102999 101.782999) (width 0.25) (layer F.Cu) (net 3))
 (segment (start 158.75 119.08) (end 158.75 132.08) (width 0.25) (layer F.Cu) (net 2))
 (via (at 158.75 132.08) (size 0.8) (drill 0.4) (layers F.Cu B.Cu) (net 2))
 (segment (start 151.11 111.44) (end 158.75 119.08) (width 0.25) (layer F.Cu) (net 2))
 (segment (start 151.11 110.49) (end 151.11 111.44) (width 0.25) (layer F.Cu) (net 2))
 (segment (start 158.75 132.08) (end 157.48 132.08) (width 0.25) (layer B.Cu) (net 2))
 (via (at 123.19 113.03) (size 0.8) (drill 0.4) (layers F.Cu B.Cu) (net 2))
 (segment (start 122.225 113.03) (end 123.19 113.03) (width 0.25) (layer B.Cu) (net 2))
 (via (at 143.51 113.03) (size 0.8) (drill 0.4) (layers F.Cu B.Cu) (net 2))
 (segment (start 123.19 113.03) (end 143.51 113.03) (width 0.25) (layer F.Cu) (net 2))
 (segment (start 151.11 110.74) (end 151.11 110.49) (width 0.25) (layer B.Cu) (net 2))
 (segment (start 148.82 113.03) (end 151.11 110.74) (width 0.25) (layer B.Cu) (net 2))
 (segment (start 143.51 113.03) (end 148.82 113.03) (width 0.25) (layer B.Cu) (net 2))
 (via (at 167.64 110.49) (size 0.8) (drill 0.4) (layers F.Cu B.Cu) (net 2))
 (segment (start 151.11 110.49) (end 167.64 110.49) (width 0.25) (layer B.Cu) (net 2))
 (via (at 181.61 113.03) (size 0.8) (drill 0.4) (layers F.Cu B.Cu) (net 2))
 (segment (start 179.07 110.49) (end 181.61 113.03) (width 0.25) (layer F.Cu) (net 2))
 (segment (start 167.64 110.49) (end 179.07 110.49) (width 0.25) (layer F.Cu) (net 2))
 (segment (start 181.61 113.03) (end 185.115 113.03) (width 0.25) (layer B.Cu) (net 2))
 (via (at 156.21 77.47) (size 0.8) (drill 0.4) (layers F.Cu B.Cu) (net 2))
 (segment (start 156.21 64.77) (end 156.21 77.47) (width 0.25) (layer B.Cu) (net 2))
 (segment (start 156.21 99.06) (end 167.64 110.49) (width 0.25) (layer F.Cu) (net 2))
 (segment (start 156.21 77.47) (end 156.21 99.06) (width 0.25) (layer F.Cu) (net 2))
 (segment (start 119.38 111.76) (end 120.65 113.03) (width 0.25) (layer B.Cu) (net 14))
 (segment (start 119.38 107.95) (end 119.38 111.76) (width 0.25) (layer B.Cu) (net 14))
 (segment (start 119.38 102.87) (end 119.38 107.95) (width 0.25) (layer B.Cu) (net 14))
 (via (at 124.46 116.84) (size 0.8) (drill 0.4) (layers F.Cu B.Cu) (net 14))
 (segment (start 120.65 113.03) (end 124.46 116.84) (width 0.25) (layer B.Cu) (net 14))
 (via (at 143.51 116.84) (size 0.8) (drill 0.4) (layers F.Cu B.Cu) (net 14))
 (segment (start 124.46 116.84) (end 143.51 116.84) (width 0.25) (layer F.Cu) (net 14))
 (segment (start 143.51 116.84) (end 149.88 116.84) (width 0.25) (layer B.Cu) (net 14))
 (segment (start 187.96 107.95) (end 187.96 102.87) (width 0.25) (layer B.Cu) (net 15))
 (segment (start 186.69 109.22) (end 187.96 107.95) (width 0.25) (layer B.Cu) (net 15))
 (segment (start 186.69 113.03) (end 186.69 109.22) (width 0.25) (layer B.Cu) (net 15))
 (via (at 167.64 116.84) (size 0.8) (drill 0.4) (layers F.Cu B.Cu) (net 15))
 (segment (start 151.13 116.84) (end 167.64 116.84) (width 0.25) (layer B.Cu) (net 15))
 (segment (start 167.64 116.84) (end 185.42 116.84) (width 0.25) (layer F.Cu) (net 15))
 (segment (start 187.96 114.3) (end 187.96 107.95) (width 0.25) (layer F.Cu) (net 15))
 (segment (start 185.42 116.84) (end 187.96 114.3) (width 0.25) (layer F.Cu) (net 15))
 (segment (start 149.86 97.79) (end 146.05 93.98) (width 0.25) (layer F.Cu) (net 22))
 (segment (start 146.05 72.39) (end 148.650001 69.789999) (width 0.25) (layer F.Cu) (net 22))
 (segment (start 146.05 93.98) (end 146.05 72.39) (width 0.25) (layer F.Cu) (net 22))
 (segment (start 153.730001 69.789999) (end 148.650001 69.789999) (width 0.25) (layer F.Cu) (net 22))
 (segment (start 153.730001 65.674999) (end 154.635 64.77) (width 0.25) (layer B.Cu) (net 22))
 (segment (start 153.730001 69.789999) (end 153.730001 65.674999) (width 0.25) (layer B.Cu) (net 22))
 (segment (start 153.580001 134.404999) (end 155.905 132.08) (width 0.25) (layer B.Cu) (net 1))
 (segment (start 153.580001 135.829999) (end 153.580001 134.404999) (width 0.25) (layer B.Cu) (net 1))
 (segment (start 148.500001 135.829999) (end 153.580001 135.829999) (width 0.25) (layer B.Cu) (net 1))
 (segment (start 156.604999 132.805001) (end 153.580001 135.829999) (width 0.25) (layer F.Cu) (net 1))
 (segment (start 151.11 97.79) (end 151.11 98.04) (width 0.25) (layer F.Cu) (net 1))
 (segment (start 159.098001 132.805001) (end 156.604999 132.805001) (width 0.25) (layer F.Cu) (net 1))
 (segment (start 159.475001 106.405001) (end 159.475001 132.428001) (width 0.25) (layer F.Cu) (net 1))
 (segment (start 159.475001 132.428001) (end 159.098001 132.805001) (width 0.25) (layer F.Cu) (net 1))
 (segment (start 151.11 98.04) (end 159.475001 106.405001) (width 0.25) (layer F.Cu) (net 1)))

